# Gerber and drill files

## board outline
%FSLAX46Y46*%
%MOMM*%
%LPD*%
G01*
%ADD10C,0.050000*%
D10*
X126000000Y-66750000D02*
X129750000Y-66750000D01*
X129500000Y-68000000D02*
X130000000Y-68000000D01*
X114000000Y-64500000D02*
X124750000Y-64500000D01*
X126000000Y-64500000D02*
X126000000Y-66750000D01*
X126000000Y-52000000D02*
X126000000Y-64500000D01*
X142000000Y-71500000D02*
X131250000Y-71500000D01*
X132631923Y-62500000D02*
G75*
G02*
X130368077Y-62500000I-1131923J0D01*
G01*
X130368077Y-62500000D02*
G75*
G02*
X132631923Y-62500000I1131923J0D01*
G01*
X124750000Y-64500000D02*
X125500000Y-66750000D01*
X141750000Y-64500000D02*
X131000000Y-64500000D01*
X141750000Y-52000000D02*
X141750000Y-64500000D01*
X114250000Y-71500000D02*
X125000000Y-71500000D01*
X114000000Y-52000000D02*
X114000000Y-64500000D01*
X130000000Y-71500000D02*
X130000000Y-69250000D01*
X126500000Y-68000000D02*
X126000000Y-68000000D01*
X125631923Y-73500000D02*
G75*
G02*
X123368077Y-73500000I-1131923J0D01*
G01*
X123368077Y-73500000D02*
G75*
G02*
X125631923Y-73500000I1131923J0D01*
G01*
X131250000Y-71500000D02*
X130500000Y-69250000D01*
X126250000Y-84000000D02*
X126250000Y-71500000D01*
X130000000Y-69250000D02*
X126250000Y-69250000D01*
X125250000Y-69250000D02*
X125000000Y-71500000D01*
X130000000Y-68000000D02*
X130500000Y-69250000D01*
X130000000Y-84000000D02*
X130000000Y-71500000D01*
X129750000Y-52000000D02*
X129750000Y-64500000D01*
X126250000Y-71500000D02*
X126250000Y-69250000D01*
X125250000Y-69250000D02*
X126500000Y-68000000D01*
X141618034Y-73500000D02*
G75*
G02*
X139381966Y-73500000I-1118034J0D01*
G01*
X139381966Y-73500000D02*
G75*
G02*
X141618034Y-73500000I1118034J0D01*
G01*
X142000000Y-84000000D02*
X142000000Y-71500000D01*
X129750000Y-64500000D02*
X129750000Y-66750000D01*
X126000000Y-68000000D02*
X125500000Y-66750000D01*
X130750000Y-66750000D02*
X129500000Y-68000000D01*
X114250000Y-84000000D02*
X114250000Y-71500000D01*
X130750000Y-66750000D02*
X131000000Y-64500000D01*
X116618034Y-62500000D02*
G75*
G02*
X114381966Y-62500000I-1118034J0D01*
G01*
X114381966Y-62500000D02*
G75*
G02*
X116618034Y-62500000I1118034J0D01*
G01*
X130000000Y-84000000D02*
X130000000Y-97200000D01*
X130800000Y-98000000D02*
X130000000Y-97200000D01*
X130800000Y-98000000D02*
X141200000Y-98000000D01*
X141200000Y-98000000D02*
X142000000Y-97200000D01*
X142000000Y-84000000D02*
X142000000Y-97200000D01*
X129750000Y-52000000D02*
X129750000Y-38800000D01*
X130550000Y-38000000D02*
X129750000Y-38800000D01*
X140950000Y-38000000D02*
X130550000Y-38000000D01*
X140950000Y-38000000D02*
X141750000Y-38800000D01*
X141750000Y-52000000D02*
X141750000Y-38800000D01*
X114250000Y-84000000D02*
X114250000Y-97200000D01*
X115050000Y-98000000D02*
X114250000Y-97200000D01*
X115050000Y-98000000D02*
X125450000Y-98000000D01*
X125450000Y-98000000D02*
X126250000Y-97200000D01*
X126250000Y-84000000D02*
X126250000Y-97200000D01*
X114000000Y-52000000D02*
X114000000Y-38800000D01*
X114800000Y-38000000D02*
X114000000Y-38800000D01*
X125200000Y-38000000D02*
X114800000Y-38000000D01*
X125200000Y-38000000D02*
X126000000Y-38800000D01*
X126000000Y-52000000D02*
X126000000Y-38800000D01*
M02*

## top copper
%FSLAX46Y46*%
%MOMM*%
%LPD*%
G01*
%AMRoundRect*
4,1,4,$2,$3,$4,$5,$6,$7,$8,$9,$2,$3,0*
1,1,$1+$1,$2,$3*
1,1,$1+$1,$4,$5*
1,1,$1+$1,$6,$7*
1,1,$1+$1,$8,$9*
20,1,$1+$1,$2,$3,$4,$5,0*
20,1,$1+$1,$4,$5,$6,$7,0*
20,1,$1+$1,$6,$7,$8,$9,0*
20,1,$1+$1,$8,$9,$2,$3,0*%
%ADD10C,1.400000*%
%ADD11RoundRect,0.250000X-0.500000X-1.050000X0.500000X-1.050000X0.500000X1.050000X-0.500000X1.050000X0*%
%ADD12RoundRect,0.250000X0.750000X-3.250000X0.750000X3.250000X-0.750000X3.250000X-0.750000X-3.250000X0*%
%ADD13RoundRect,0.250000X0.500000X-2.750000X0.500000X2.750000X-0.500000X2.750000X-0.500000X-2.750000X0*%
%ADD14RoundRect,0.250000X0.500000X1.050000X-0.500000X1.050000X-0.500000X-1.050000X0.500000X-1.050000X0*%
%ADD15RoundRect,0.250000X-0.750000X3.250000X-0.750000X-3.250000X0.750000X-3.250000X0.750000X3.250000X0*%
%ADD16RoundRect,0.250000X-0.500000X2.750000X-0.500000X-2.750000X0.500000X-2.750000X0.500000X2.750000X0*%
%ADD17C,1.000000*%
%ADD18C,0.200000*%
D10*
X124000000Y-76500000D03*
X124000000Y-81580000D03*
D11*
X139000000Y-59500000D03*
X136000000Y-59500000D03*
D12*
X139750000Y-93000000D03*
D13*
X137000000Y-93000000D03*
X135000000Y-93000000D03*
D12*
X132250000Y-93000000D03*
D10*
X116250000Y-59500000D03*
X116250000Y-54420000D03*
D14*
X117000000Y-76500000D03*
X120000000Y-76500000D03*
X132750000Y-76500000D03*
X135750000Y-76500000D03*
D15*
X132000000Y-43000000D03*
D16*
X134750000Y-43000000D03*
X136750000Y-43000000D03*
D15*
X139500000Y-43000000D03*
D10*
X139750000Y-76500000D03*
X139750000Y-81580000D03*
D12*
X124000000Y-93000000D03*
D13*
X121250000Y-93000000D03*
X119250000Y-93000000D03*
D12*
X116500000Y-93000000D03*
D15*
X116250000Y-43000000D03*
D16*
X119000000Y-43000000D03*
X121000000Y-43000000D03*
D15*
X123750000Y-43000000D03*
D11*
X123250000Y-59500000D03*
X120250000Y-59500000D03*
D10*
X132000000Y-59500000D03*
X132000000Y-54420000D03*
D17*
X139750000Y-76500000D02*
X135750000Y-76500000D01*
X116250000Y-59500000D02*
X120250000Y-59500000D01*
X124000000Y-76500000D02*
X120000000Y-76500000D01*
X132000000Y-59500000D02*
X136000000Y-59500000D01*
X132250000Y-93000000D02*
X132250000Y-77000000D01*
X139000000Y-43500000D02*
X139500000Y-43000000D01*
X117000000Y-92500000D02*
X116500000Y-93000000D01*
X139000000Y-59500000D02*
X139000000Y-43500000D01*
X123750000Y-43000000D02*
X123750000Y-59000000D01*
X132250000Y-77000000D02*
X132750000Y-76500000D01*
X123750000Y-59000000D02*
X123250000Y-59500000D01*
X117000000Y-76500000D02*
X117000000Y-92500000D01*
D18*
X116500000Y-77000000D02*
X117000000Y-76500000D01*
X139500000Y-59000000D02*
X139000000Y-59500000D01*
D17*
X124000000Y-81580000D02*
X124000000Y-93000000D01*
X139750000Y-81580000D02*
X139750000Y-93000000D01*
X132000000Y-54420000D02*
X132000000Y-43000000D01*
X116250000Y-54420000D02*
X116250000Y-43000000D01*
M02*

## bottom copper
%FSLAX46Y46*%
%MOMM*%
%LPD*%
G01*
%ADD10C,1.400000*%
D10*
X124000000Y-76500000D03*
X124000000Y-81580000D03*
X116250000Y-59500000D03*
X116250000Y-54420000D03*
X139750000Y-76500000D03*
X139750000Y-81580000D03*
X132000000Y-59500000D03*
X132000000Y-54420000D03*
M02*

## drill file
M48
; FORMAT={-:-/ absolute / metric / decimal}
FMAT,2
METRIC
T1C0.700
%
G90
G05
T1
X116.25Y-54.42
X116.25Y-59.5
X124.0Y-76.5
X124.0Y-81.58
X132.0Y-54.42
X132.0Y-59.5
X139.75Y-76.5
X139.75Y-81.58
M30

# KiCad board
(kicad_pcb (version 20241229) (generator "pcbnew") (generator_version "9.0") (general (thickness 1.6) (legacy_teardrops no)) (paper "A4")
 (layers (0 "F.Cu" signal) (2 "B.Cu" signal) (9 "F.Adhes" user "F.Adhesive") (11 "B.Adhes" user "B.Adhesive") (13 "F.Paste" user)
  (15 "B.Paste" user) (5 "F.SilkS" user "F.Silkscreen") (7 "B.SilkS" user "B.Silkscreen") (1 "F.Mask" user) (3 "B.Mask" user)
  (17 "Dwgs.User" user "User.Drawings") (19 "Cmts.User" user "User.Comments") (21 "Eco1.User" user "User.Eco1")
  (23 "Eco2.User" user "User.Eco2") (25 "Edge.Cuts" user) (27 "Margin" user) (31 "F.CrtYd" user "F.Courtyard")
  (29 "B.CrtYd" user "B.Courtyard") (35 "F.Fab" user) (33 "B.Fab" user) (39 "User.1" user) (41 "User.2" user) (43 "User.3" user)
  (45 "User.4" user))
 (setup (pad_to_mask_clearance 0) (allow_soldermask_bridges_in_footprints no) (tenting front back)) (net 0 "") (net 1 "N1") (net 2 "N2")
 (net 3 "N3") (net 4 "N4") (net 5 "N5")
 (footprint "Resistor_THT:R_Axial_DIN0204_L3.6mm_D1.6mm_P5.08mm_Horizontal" (layer "F.Cu") (at 124 76.5 -90)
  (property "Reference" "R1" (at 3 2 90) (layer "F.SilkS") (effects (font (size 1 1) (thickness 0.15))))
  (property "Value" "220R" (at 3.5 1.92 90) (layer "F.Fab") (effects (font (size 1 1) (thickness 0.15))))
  (pad "1" thru_hole circle (at 0 0 270) (size 1.4 1.4) (drill 0.7) (layers "*.Cu" "*.Mask") (remove_unused_layers no) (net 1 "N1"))
  (pad "2" thru_hole circle (at 5.08 0 270) (size 1.4 1.4) (drill 0.7) (layers "*.Cu" "*.Mask") (remove_unused_layers no) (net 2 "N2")))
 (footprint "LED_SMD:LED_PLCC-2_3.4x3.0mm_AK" (layer "F.Cu") (at 137.5 59.5)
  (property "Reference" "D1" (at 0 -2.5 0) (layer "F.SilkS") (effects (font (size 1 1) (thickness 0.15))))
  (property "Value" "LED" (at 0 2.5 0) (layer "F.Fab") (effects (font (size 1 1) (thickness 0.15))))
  (pad "1" smd roundrect (at 1.5 0) (size 1.5 2.6) (layers "F.Cu" "F.Mask" "F.Paste") (roundrect_rratio 0.1666666667) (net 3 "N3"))
  (pad "2" smd roundrect (at -1.5 0) (size 1.5 2.6) (layers "F.Cu" "F.Mask" "F.Paste") (roundrect_rratio 0.1666666667) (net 1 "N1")))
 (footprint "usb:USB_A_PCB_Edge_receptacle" (layer "F.Cu") (at 136 93 90)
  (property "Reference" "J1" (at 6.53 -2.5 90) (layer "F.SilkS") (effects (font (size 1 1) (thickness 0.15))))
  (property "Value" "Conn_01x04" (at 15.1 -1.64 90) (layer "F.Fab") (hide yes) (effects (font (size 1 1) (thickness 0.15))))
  (fp_line (start 9 -6) (end -4.2 -6) (stroke (width 0.05) (type default)) (layer "Edge.Cuts"))
  (fp_line (start -5 -5.2) (end -4.2 -6) (stroke (width 0.05) (type default)) (layer "Edge.Cuts"))
  (fp_line (start -5 -5.2) (end -5 5.2) (stroke (width 0.05) (type default)) (layer "Edge.Cuts"))
  (fp_line (start -5 5.2) (end -4.2 6) (stroke (width 0.05) (type default)) (layer "Edge.Cuts"))
  (fp_line (start 9 6) (end -4.2 6) (stroke (width 0.05) (type default)) (layer "Edge.Cuts"))
  (pad "1" smd roundrect (at 0 3.75 90) (size 7 2) (layers "F.Cu" "F.Mask") (roundrect_rratio 0.125) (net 2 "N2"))
  (pad "2" smd roundrect (at 0 1 90) (size 6 1.5) (layers "F.Cu" "F.Mask") (roundrect_rratio 0.1666666667) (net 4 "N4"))
  (pad "3" smd roundrect (at 0 -1 90) (size 6 1.5) (layers "F.Cu" "F.Mask") (roundrect_rratio 0.1666666667) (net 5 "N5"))
  (pad "4" smd roundrect (at 0 -3.75 90) (size 7 2) (layers "F.Cu" "F.Mask") (roundrect_rratio 0.125) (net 3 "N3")))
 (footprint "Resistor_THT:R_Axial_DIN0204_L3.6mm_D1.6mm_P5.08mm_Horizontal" (layer "F.Cu") (at 116.25 59.5 90)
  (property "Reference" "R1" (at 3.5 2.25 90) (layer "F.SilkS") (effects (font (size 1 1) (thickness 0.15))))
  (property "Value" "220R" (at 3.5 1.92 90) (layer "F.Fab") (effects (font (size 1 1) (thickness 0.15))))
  (pad "1" thru_hole circle (at 0 0 90) (size 1.4 1.4) (drill 0.7) (layers "*.Cu" "*.Mask") (remove_unused_layers no) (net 1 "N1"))
  (pad "2" thru_hole circle (at 5.08 0 90) (size 1.4 1.4) (drill 0.7) (layers "*.Cu" "*.Mask") (remove_unused_layers no) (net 2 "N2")))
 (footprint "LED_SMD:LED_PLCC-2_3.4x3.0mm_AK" (layer "F.Cu") (at 118.5 76.5 180)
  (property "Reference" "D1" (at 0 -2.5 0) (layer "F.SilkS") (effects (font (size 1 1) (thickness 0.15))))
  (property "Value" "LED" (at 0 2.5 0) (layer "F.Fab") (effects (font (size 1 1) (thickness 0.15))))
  (pad "1" smd roundrect (at 1.5 0 180) (size 1.5 2.6) (layers "F.Cu" "F.Mask" "F.Paste") (roundrect_rratio 0.1666666667) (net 3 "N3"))
  (pad "2" smd roundrect (at -1.5 0 180) (size 1.5 2.6) (layers "F.Cu" "F.Mask" "F.Paste") (roundrect_rratio 0.1666666667) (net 1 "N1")))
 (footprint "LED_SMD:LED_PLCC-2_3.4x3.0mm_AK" (layer "F.Cu") (at 134.25 76.5 180)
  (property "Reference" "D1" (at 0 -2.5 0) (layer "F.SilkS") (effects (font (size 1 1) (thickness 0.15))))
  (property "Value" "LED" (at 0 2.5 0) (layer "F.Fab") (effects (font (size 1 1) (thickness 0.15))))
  (pad "1" smd roundrect (at 1.5 0 180) (size 1.5 2.6) (layers "F.Cu" "F.Mask" "F.Paste") (roundrect_rratio 0.1666666667) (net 3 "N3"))
  (pad "2" smd roundrect (at -1.5 0 180) (size 1.5 2.6) (layers "F.Cu" "F.Mask" "F.Paste") (roundrect_rratio 0.1666666667) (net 1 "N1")))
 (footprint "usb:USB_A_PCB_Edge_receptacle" (layer "F.Cu") (at 135.75 43 -90)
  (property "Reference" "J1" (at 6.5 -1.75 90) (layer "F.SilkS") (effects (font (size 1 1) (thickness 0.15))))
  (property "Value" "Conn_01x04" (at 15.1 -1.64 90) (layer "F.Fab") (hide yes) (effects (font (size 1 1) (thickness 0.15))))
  (fp_line (start 9 6) (end -4.2 6) (stroke (width 0.05) (type default)) (layer "Edge.Cuts") (net 1))
  (fp_line (start -5 5.2) (end -4.2 6) (stroke (width 0.05) (type default)) (layer "Edge.Cuts") (net 1))
  (fp_line (start -5 -5.2) (end -5 5.2) (stroke (width 0.05) (type default)) (layer "Edge.Cuts") (net 1))
  (fp_line (start -5 -5.2) (end -4.2 -6) (stroke (width 0.05) (type default)) (layer "Edge.Cuts") (net 1))
  (fp_line (start 9 -6) (end -4.2 -6) (stroke (width 0.05) (type default)) (layer "Edge.Cuts") (net 1))
  (pad "1" smd roundrect (at 0 3.75 270) (size 7 2) (layers "F.Cu" "F.Mask") (roundrect_rratio 0.125) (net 2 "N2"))
  (pad "2" smd roundrect (at 0 1 270) (size 6 1.5) (layers "F.Cu" "F.Mask") (roundrect_rratio 0.1666666667) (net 4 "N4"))
  (pad "3" smd roundrect (at 0 -1 270) (size 6 1.5) (layers "F.Cu" "F.Mask") (roundrect_rratio 0.1666666667) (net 5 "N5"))
  (pad "4" smd roundrect (at 0 -3.75 270) (size 7 2) (layers "F.Cu" "F.Mask") (roundrect_rratio 0.125) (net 3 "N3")))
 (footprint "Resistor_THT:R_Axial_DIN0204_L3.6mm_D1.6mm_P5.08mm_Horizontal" (layer "F.Cu") (at 139.75 76.5 -90)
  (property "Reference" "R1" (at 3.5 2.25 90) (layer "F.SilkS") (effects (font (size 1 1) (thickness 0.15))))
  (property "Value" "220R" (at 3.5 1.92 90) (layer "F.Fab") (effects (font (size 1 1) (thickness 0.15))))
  (pad "1" thru_hole circle (at 0 0 270) (size 1.4 1.4) (drill 0.7) (layers "*.Cu" "*.Mask") (remove_unused_layers no) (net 1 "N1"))
  (pad "2" thru_hole circle (at 5.08 0 270) (size 1.4 1.4) (drill 0.7) (layers "*.Cu" "*.Mask") (remove_unused_layers no) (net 2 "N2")))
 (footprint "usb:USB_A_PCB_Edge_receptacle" (layer "F.Cu") (at 120.25 93 90)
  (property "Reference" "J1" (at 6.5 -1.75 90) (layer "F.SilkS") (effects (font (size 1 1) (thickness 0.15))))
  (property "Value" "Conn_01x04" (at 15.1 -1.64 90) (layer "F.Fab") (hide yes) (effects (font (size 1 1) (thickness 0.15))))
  (fp_line (start 9 -6) (end -4.2 -6) (stroke (width 0.05) (type default)) (layer "Edge.Cuts"))
  (fp_line (start -5 -5.2) (end -4.2 -6) (stroke (width 0.05) (type default)) (layer "Edge.Cuts"))
  (fp_line (start -5 -5.2) (end -5 5.2) (stroke (width 0.05) (type default)) (layer "Edge.Cuts"))
  (fp_line (start -5 5.2) (end -4.2 6) (stroke (width 0.05) (type default)) (layer "Edge.Cuts"))
  (fp_line (start 9 6) (end -4.2 6) (stroke (width 0.05) (type default)) (layer "Edge.Cuts"))
  (pad "1" smd roundrect (at 0 3.75 90) (size 7 2) (layers "F.Cu" "F.Mask") (roundrect_rratio 0.125) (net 2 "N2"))
  (pad "2" smd roundrect (at 0 1 90) (size 6 1.5) (layers "F.Cu" "F.Mask") (roundrect_rratio 0.1666666667) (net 4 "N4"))
  (pad "3" smd roundrect (at 0 -1 90) (size 6 1.5) (layers "F.Cu" "F.Mask") (roundrect_rratio 0.1666666667) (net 5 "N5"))
  (pad "4" smd roundrect (at 0 -3.75 90) (size 7 2) (layers "F.Cu" "F.Mask") (roundrect_rratio 0.125) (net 3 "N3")))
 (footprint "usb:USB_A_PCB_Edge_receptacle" (layer "F.Cu") (at 120 43 -90)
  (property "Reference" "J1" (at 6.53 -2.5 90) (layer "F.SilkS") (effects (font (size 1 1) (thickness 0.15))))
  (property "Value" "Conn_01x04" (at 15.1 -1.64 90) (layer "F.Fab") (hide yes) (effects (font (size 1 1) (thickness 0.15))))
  (fp_line (start 9 6) (end -4.2 6) (stroke (width 0.05) (type default)) (layer "Edge.Cuts") (net 1))
  (fp_line (start -5 5.2) (end -4.2 6) (stroke (width 0.05) (type default)) (layer "Edge.Cuts") (net 1))
  (fp_line (start -5 -5.2) (end -5 5.2) (stroke (width 0.05) (type default)) (layer "Edge.Cuts") (net 1))
  (fp_line (start -5 -5.2) (end -4.2 -6) (stroke (width 0.05) (type default)) (layer "Edge.Cuts") (net 1))
  (fp_line (start 9 -6) (end -4.2 -6) (stroke (width 0.05) (type default)) (layer "Edge.Cuts") (net 1))
  (pad "1" smd roundrect (at 0 3.75 270) (size 7 2) (layers "F.Cu" "F.Mask") (roundrect_rratio 0.125) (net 2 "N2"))
  (pad "2" smd roundrect (at 0 1 270) (size 6 1.5) (layers "F.Cu" "F.Mask") (roundrect_rratio 0.1666666667) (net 4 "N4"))
  (pad "3" smd roundrect (at 0 -1 270) (size 6 1.5) (layers "F.Cu" "F.Mask") (roundrect_rratio 0.1666666667) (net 5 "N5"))
  (pad "4" smd roundrect (at 0 -3.75 270) (size 7 2) (layers "F.Cu" "F.Mask") (roundrect_rratio 0.125) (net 3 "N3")))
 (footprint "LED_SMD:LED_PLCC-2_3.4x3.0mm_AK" (layer "F.Cu") (at 121.75 59.5)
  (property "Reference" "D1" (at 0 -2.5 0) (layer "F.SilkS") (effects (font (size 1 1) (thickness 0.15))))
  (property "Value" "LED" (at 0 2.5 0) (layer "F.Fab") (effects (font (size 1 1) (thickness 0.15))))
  (pad "1" smd roundrect (at 1.5 0) (size 1.5 2.6) (layers "F.Cu" "F.Mask" "F.Paste") (roundrect_rratio 0.1666666667) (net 3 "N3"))
  (pad "2" smd roundrect (at -1.5 0) (size 1.5 2.6) (layers "F.Cu" "F.Mask" "F.Paste") (roundrect_rratio 0.1666666667) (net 1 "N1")))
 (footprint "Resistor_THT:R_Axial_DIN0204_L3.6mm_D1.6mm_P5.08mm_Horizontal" (layer "F.Cu") (at 132 59.5 90)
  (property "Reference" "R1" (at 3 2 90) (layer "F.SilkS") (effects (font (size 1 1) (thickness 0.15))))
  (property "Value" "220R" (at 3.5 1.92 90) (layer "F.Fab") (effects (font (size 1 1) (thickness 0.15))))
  (pad "1" thru_hole circle (at 0 0 90) (size 1.4 1.4) (drill 0.7) (layers "*.Cu" "*.Mask") (remove_unused_layers no) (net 1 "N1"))
  (pad "2" thru_hole circle (at 5.08 0 90) (size 1.4 1.4) (drill 0.7) (layers "*.Cu" "*.Mask") (remove_unused_layers no) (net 2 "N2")))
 (gr_line (start 126 66.75) (end 129.75 66.75) (stroke (width 0.05) (type default)) (layer "Edge.Cuts"))
 (gr_line (start 129.5 68) (end 130 68) (stroke (width 0.05) (type default)) (layer "Edge.Cuts"))
 (gr_line (start 114 64.5) (end 124.75 64.5) (stroke (width 0.05) (type default)) (layer "Edge.Cuts"))
 (gr_line (start 126 64.5) (end 126 66.75) (stroke (width 0.05) (type default)) (layer "Edge.Cuts"))
 (gr_line (start 126 52) (end 126 64.5) (stroke (width 0.05) (type default)) (layer "Edge.Cuts"))
 (gr_line (start 142 71.5) (end 131.25 71.5) (stroke (width 0.05) (type default)) (layer "Edge.Cuts"))
 (gr_circle (center 131.5 62.5) (end 131.375 63.625) (stroke (width 0.05) (type default)) (fill no) (layer "Edge.Cuts"))
 (gr_line (start 124.75 64.5) (end 125.5 66.75) (stroke (width 0.05) (type default)) (layer "Edge.Cuts"))
 (gr_line (start 141.75 64.5) (end 131 64.5) (stroke (width 0.05) (type default)) (layer "Edge.Cuts"))
 (gr_line (start 141.75 52) (end 141.75 64.5) (stroke (width 0.05) (type default)) (layer "Edge.Cuts"))
 (gr_line (start 114.25 71.5) (end 125 71.5) (stroke (width 0.05) (type default)) (layer "Edge.Cuts"))
 (gr_line (start 114 52) (end 114 64.5) (stroke (width 0.05) (type default)) (layer "Edge.Cuts"))
 (gr_line (start 130 71.5) (end 130 69.25) (stroke (width 0.05) (type default)) (layer "Edge.Cuts"))
 (gr_line (start 126.5 68) (end 126 68) (stroke (width 0.05) (type default)) (layer "Edge.Cuts"))
 (gr_circle (center 124.5 73.5) (end 124.625 72.375) (stroke (width 0.05) (type default)) (fill no) (layer "Edge.Cuts"))
 (gr_line (start 131.25 71.5) (end 130.5 69.25) (stroke (width 0.05) (type default)) (layer "Edge.Cuts"))
 (gr_line (start 126.25 84) (end 126.25 71.5) (stroke (width 0.05) (type default)) (layer "Edge.Cuts"))
 (gr_line (start 130 69.25) (end 126.25 69.25) (stroke (width 0.05) (type default)) (layer "Edge.Cuts"))
 (gr_line (start 125.25 69.25) (end 125 71.5) (stroke (width 0.05) (type default)) (layer "Edge.Cuts"))
 (gr_line (start 130 68) (end 130.5 69.25) (stroke (width 0.05) (type default)) (layer "Edge.Cuts"))
 (gr_line (start 130 84) (end 130 71.5) (stroke (width 0.05) (type default)) (layer "Edge.Cuts"))
 (gr_line (start 129.75 52) (end 129.75 64.5) (stroke (width 0.05) (type default)) (layer "Edge.Cuts"))
 (gr_line (start 126.25 71.5) (end 126.25 69.25) (stroke (width 0.05) (type default)) (layer "Edge.Cuts"))
 (gr_line (start 125.25 69.25) (end 126.5 68) (stroke (width 0.05) (type default)) (layer "Edge.Cuts"))
 (gr_circle (center 140.5 73.5) (end 140 72.5) (stroke (width 0.05) (type default)) (fill no) (layer "Edge.Cuts"))
 (gr_line (start 142 84) (end 142 71.5) (stroke (width 0.05) (type default)) (layer "Edge.Cuts"))
 (gr_line (start 129.75 64.5) (end 129.75 66.75) (stroke (width 0.05) (type default)) (layer "Edge.Cuts"))
 (gr_line (start 126 68) (end 125.5 66.75) (stroke (width 0.05) (type default)) (layer "Edge.Cuts"))
 (gr_line (start 130.75 66.75) (end 129.5 68) (stroke (width 0.05) (type default)) (layer "Edge.Cuts"))
 (gr_line (start 114.25 84) (end 114.25 71.5) (stroke (width 0.05) (type default)) (layer "Edge.Cuts"))
 (gr_line (start 130.75 66.75) (end 131 64.5) (stroke (width 0.05) (type default)) (layer "Edge.Cuts"))
 (gr_circle (center 115.5 62.5) (end 116 63.5) (stroke (width 0.05) (type default)) (fill no) (layer "Edge.Cuts"))
 (segment (start 139.75 76.5) (end 135.75 76.5) (width 1) (layer "F.Cu") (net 1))
 (segment (start 116.25 59.5) (end 120.25 59.5) (width 1) (layer "F.Cu") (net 1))
 (segment (start 124 76.5) (end 120 76.5) (width 1) (layer "F.Cu") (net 1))
 (segment (start 132 59.5) (end 136 59.5) (width 1) (layer "F.Cu") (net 1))
 (segment (start 132.25 93) (end 132.25 77) (width 1) (layer "F.Cu") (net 3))
 (segment (start 139 43.5) (end 139.5 43) (width 1) (layer "F.Cu") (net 3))
 (segment (start 117 92.5) (end 116.5 93) (width 1) (layer "F.Cu") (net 3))
 (segment (start 139 59.5) (end 139 43.5) (width 1) (layer "F.Cu") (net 3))
 (segment (start 123.75 43) (end 123.75 59) (width 1) (layer "F.Cu") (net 3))
 (segment (start 132.25 77) (end 132.75 76.5) (width 1) (layer "F.Cu") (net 3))
 (segment (start 123.75 59) (end 123.25 59.5) (width 1) (layer "F.Cu") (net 3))
 (segment (start 117 76.5) (end 117 92.5) (width 1) (layer "F.Cu") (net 3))
 (segment (start 116.5 77) (end 117 76.5) (width 0.2) (layer "F.Cu") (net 3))
 (segment (start 139.5 59) (end 139 59.5) (width 0.2) (layer "F.Cu") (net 3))
 (segment (start 124 81.58) (end 124 93) (width 1) (layer "F.Cu") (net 2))
 (segment (start 139.75 81.58) (end 139.75 93) (width 1) (layer "F.Cu") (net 2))
 (segment (start 132 54.42) (end 132 43) (width 1) (layer "F.Cu") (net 2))
 (segment (start 116.25 54.42) (end 116.25 43) (width 1) (layer "F.Cu") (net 2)))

